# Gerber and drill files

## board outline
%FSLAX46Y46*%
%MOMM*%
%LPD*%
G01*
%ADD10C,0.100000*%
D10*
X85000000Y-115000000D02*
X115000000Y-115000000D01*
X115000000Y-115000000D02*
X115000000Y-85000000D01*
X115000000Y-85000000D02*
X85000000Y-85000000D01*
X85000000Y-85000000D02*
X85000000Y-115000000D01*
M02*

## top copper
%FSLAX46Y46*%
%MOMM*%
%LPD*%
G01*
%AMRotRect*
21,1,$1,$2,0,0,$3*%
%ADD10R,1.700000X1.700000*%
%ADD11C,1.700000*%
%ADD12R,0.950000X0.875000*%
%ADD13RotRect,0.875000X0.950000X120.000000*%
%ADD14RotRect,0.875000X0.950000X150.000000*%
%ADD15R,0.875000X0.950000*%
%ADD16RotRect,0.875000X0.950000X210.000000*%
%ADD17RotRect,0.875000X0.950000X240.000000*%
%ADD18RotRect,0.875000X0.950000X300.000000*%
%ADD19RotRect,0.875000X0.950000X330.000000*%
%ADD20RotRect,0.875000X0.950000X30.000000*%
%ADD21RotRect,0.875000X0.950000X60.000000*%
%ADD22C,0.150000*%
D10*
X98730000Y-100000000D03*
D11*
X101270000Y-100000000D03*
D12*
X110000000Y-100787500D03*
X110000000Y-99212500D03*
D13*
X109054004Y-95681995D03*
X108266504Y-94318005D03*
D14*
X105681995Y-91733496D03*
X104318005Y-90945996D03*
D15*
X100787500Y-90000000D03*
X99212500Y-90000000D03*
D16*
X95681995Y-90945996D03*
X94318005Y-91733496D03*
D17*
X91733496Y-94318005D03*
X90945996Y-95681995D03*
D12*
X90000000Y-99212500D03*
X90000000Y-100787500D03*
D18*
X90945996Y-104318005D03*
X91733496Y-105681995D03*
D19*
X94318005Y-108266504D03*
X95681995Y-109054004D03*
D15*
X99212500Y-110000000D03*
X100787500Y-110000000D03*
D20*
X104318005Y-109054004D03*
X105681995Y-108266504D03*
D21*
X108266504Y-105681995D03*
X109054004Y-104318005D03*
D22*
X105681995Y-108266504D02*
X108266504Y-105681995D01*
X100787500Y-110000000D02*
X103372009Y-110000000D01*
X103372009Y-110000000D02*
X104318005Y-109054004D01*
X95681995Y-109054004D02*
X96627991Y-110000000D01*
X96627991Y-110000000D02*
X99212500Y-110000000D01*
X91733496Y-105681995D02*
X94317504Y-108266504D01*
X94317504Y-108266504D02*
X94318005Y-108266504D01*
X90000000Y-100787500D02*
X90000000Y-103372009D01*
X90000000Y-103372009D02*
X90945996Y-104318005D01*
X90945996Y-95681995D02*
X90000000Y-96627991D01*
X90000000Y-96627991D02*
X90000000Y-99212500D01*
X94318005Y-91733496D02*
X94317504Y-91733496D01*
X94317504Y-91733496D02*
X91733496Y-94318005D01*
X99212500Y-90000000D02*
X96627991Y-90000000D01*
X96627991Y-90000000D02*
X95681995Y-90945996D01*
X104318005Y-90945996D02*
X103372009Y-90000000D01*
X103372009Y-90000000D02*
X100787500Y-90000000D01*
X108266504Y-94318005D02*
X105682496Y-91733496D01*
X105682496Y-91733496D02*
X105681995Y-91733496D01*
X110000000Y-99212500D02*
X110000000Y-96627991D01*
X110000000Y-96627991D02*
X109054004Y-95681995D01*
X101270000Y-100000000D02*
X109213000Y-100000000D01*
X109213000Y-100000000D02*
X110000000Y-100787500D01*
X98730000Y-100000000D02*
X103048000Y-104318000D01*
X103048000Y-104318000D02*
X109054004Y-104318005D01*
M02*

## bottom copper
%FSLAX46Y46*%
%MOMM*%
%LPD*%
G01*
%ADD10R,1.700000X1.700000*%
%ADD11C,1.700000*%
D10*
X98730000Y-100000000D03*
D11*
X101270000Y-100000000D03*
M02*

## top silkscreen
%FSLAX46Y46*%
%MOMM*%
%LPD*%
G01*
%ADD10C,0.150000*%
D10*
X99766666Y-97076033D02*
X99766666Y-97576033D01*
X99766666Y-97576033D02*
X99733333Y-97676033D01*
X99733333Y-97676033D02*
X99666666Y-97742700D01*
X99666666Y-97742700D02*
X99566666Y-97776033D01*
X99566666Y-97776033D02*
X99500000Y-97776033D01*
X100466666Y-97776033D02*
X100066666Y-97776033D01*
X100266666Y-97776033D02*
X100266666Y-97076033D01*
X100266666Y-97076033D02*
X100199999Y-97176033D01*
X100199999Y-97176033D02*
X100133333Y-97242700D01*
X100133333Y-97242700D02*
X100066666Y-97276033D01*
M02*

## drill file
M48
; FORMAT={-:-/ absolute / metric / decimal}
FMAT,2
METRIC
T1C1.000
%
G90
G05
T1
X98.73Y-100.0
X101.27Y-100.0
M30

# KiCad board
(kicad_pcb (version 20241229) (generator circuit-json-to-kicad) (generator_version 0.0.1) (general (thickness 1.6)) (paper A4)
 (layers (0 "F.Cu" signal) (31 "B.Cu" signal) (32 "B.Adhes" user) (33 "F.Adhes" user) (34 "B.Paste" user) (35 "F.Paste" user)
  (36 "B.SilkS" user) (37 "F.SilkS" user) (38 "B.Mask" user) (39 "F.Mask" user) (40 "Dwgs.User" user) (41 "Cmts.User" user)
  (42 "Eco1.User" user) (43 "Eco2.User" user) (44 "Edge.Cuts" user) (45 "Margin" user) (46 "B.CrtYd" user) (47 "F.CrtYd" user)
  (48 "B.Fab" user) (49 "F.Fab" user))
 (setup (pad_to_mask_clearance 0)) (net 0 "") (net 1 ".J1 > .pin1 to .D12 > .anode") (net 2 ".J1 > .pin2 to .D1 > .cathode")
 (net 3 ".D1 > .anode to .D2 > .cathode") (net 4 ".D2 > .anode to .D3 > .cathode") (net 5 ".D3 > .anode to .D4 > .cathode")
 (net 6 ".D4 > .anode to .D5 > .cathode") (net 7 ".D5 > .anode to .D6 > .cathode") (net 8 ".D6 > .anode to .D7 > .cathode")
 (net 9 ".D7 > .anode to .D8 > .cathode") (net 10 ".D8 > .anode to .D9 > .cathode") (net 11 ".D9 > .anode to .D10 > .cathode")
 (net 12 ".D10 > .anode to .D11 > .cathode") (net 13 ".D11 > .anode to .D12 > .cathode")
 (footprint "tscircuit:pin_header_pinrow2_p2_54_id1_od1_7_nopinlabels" (layer F.Cu) (at 100 100 0)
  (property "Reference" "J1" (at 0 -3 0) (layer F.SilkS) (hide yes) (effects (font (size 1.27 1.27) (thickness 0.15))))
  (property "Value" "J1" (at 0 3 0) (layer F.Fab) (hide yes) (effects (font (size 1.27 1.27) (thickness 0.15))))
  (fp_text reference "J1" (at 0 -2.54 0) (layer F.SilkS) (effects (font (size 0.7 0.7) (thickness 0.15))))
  (pad "1" thru_hole rect (at -1.27 0 0) (size 1.7 1.7) (drill 1) (layers *.Cu *.Mask) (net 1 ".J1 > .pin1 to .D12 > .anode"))
  (pad "2" thru_hole circle (at 1.27 0 0) (size 1.7 1.7) (drill 1) (layers *.Cu *.Mask) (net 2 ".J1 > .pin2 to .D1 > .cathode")))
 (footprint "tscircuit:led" (layer F.Cu) (at 110 100 90)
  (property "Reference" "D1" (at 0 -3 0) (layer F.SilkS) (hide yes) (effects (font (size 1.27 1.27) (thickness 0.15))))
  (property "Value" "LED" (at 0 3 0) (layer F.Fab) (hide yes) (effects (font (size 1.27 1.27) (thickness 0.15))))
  (pad "2" smd rect (at -0.7875 0 0) (size 0.95 0.875) (layers F.Cu F.Mask) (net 2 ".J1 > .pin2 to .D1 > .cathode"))
  (pad "1" smd rect (at 0.7875 0 0) (size 0.95 0.875) (layers F.Cu F.Mask) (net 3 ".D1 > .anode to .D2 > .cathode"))
  (pad "" smd rect (at -0.7875 0 0) (size 0.6649999999999999 0.6124999999999999) (layers F.Paste))
  (pad "" smd rect (at 0.7875 0 0) (size 0.6649999999999999 0.6124999999999999) (layers F.Paste)))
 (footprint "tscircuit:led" (layer F.Cu) (at 108.66025403784438 95 120)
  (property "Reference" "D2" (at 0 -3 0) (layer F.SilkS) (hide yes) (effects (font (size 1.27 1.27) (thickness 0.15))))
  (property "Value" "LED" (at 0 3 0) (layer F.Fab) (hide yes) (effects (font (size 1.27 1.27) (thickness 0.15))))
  (pad "2" smd rect (at -0.7874999999999996 0 120) (size 0.875 0.95) (layers F.Cu F.Mask) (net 3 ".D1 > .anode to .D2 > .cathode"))
  (pad "1" smd rect (at 0.7874999999999988 1.7763568394002505e-15 120) (size 0.875 0.95) (layers F.Cu F.Mask)
   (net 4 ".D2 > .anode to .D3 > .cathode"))
  (pad "" smd rect (at -0.7874999999999996 0 120) (size 0.6124999999999999 0.6649999999999999) (layers F.Paste))
  (pad "" smd rect (at 0.7874999999999988 1.7763568394002505e-15 120) (size 0.6124999999999999 0.6649999999999999) (layers F.Paste)))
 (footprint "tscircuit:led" (layer F.Cu) (at 105 91.33974596215562 150)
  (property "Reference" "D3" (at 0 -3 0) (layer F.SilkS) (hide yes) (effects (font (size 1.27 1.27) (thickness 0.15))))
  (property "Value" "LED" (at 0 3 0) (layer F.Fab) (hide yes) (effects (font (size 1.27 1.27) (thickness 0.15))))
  (pad "2" smd rect (at -0.7874999999999996 -1.7763568394002505e-15 150) (size 0.875 0.95) (layers F.Cu F.Mask)
   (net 4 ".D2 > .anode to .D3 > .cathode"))
  (pad "1" smd rect (at 0.7875000000000005 0 150) (size 0.875 0.95) (layers F.Cu F.Mask) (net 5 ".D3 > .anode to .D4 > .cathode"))
  (pad "" smd rect (at -0.7874999999999996 -1.7763568394002505e-15 150) (size 0.6124999999999999 0.6649999999999999) (layers F.Paste))
  (pad "" smd rect (at 0.7875000000000005 0 150) (size 0.6124999999999999 0.6649999999999999) (layers F.Paste)))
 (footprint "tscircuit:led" (layer F.Cu) (at 100 90 180)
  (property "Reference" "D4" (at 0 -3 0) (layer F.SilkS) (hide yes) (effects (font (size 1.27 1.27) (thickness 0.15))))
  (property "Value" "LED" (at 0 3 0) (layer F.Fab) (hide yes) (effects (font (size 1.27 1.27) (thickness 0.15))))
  (pad "2" smd rect (at -0.7875000000000001 0 0) (size 0.875 0.95) (layers F.Cu F.Mask) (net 5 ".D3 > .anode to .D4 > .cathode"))
  (pad "1" smd rect (at 0.7874999999999999 0 0) (size 0.875 0.95) (layers F.Cu F.Mask) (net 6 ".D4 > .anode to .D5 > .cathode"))
  (pad "" smd rect (at -0.7875000000000001 0 0) (size 0.6124999999999999 0.6649999999999999) (layers F.Paste))
  (pad "" smd rect (at 0.7874999999999999 0 0) (size 0.6124999999999999 0.6649999999999999) (layers F.Paste)))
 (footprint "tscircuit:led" (layer F.Cu) (at 95 91.3397459621556 209.99999999999997)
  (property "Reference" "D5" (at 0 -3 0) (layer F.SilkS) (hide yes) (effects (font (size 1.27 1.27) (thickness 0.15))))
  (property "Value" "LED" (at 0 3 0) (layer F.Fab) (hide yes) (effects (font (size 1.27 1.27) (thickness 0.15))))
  (pad "2" smd rect
   (at -0.7875000000000005 1.7763568394002505e-15 209.99999999999997) (size 0.875 0.95) (layers F.Cu F.Mask)
   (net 6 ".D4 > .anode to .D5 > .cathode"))
  (pad "1" smd rect
   (at 0.7875000000000005 -1.7763568394002505e-15 209.99999999999997) (size 0.875 0.95) (layers F.Cu F.Mask)
   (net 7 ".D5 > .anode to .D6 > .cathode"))
  (pad "" smd rect
   (at -0.7875000000000005 1.7763568394002505e-15 209.99999999999997) (size 0.6124999999999999 0.6649999999999999) (layers F.Paste))
  (pad "" smd rect
   (at 0.7875000000000005 -1.7763568394002505e-15 209.99999999999997) (size 0.6124999999999999 0.6649999999999999) (layers F.Paste)))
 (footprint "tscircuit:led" (layer F.Cu) (at 91.33974596215562 95 239.99999999999994)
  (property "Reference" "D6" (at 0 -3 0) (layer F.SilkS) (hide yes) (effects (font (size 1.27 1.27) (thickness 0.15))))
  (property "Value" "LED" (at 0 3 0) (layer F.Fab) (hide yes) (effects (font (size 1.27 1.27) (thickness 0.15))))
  (pad "2" smd rect (at -0.7875000000000005 0 239.99999999999994) (size 0.875 0.95) (layers F.Cu F.Mask)
   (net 7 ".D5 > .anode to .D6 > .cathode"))
  (pad "1" smd rect (at 0.7875000000000001 0 239.99999999999994) (size 0.875 0.95) (layers F.Cu F.Mask)
   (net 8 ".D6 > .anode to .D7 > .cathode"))
  (pad "" smd rect (at -0.7875000000000005 0 239.99999999999994) (size 0.6124999999999999 0.6649999999999999) (layers F.Paste))
  (pad "" smd rect (at 0.7875000000000001 0 239.99999999999994) (size 0.6124999999999999 0.6649999999999999) (layers F.Paste)))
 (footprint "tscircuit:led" (layer F.Cu) (at 90 100 270)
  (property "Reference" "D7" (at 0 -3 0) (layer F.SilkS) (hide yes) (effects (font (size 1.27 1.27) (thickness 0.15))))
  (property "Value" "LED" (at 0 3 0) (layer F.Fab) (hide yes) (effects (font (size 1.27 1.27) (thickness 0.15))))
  (pad "2" smd rect (at -0.7875 0 0) (size 0.95 0.875) (layers F.Cu F.Mask) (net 8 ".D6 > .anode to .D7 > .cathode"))
  (pad "1" smd rect (at 0.7875 0 0) (size 0.95 0.875) (layers F.Cu F.Mask) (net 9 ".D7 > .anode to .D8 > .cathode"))
  (pad "" smd rect (at -0.7875 0 0) (size 0.6649999999999999 0.6124999999999999) (layers F.Paste))
  (pad "" smd rect (at 0.7875 0 0) (size 0.6649999999999999 0.6124999999999999) (layers F.Paste)))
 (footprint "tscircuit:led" (layer F.Cu) (at 91.33974596215562 105 300)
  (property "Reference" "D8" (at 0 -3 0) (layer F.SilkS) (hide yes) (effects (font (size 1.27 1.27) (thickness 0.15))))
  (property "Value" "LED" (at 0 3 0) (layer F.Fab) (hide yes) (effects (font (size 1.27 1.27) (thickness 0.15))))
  (pad "2" smd rect (at -0.7875000000000001 0 300) (size 0.875 0.95) (layers F.Cu F.Mask) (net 9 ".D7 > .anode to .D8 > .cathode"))
  (pad "1" smd rect (at 0.7875000000000005 -1.7763568394002505e-15 300) (size 0.875 0.95) (layers F.Cu F.Mask)
   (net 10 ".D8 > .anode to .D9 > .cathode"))
  (pad "" smd rect (at -0.7875000000000001 0 300) (size 0.6124999999999999 0.6649999999999999) (layers F.Paste))
  (pad "" smd rect (at 0.7875000000000005 -1.7763568394002505e-15 300) (size 0.6124999999999999 0.6649999999999999) (layers F.Paste)))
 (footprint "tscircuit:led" (layer F.Cu) (at 95 108.66025403784438 330)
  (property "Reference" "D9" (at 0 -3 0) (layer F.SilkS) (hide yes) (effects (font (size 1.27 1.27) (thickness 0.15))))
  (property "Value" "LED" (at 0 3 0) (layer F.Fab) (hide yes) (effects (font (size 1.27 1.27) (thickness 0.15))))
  (pad "2" smd rect (at -0.7875000000000005 0 330) (size 0.875 0.95) (layers F.Cu F.Mask) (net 10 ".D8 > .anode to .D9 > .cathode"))
  (pad "1" smd rect (at 0.7875000000000005 0 330) (size 0.875 0.95) (layers F.Cu F.Mask) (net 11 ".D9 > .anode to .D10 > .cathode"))
  (pad "" smd rect (at -0.7875000000000005 0 330) (size 0.6124999999999999 0.6649999999999999) (layers F.Paste))
  (pad "" smd rect (at 0.7875000000000005 0 330) (size 0.6124999999999999 0.6649999999999999) (layers F.Paste)))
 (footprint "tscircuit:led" (layer F.Cu) (at 100 110 0)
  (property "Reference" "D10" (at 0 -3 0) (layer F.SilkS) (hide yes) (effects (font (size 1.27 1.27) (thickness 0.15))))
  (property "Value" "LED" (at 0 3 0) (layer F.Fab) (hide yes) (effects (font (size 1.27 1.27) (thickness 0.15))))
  (pad "2" smd rect (at -0.7875 0 0) (size 0.875 0.95) (layers F.Cu F.Mask) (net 11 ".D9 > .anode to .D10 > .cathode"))
  (pad "1" smd rect (at 0.7875 0 0) (size 0.875 0.95) (layers F.Cu F.Mask) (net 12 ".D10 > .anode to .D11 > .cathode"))
  (pad "" smd rect (at -0.7875 0 0) (size 0.6124999999999999 0.6649999999999999) (layers F.Paste))
  (pad "" smd rect (at 0.7875 0 0) (size 0.6124999999999999 0.6649999999999999) (layers F.Paste)))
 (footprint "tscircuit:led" (layer F.Cu) (at 105 108.66025403784438 30)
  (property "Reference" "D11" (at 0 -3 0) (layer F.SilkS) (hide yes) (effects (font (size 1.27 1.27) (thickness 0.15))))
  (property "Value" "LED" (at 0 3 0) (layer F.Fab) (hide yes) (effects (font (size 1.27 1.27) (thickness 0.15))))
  (pad "2" smd rect (at -0.7875000000000005 0 30) (size 0.875 0.95) (layers F.Cu F.Mask) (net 12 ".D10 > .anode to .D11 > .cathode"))
  (pad "1" smd rect (at 0.7875000000000005 -1.7763568394002505e-15 30) (size 0.875 0.95) (layers F.Cu F.Mask)
   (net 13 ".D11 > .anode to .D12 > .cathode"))
  (pad "" smd rect (at -0.7875000000000005 0 30) (size 0.6124999999999999 0.6649999999999999) (layers F.Paste))
  (pad "" smd rect (at 0.7875000000000005 -1.7763568394002505e-15 30) (size 0.6124999999999999 0.6649999999999999) (layers F.Paste)))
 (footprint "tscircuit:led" (layer F.Cu) (at 108.66025403784438 105 60)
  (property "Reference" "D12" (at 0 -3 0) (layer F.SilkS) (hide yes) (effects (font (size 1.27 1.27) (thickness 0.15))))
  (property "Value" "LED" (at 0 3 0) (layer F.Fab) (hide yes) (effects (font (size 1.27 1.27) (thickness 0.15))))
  (pad "2" smd rect (at -0.7874999999999996 0 60) (size 0.875 0.95) (layers F.Cu F.Mask) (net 13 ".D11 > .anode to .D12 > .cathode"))
  (pad "1" smd rect (at 0.7875000000000005 0 60) (size 0.875 0.95) (layers F.Cu F.Mask) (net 1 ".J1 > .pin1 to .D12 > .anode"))
  (pad "" smd rect (at -0.7874999999999996 0 60) (size 0.6124999999999999 0.6649999999999999) (layers F.Paste))
  (pad "" smd rect (at 0.7875000000000005 0 60) (size 0.6124999999999999 0.6649999999999999) (layers F.Paste)))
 (segment (start 105.68199500548025 108.26650403784438) (end 108.26650403784438 105.68199500548025) (width 0.15) (layer F.Cu) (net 13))
 (segment (start 100.7875 110) (end 103.37200903236415 110) (width 0.15) (layer F.Cu) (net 12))
 (segment (start 103.37200903236415 110) (end 104.31800499451975 109.05400403784438) (width 0.15) (layer F.Cu) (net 12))
 (segment (start 95.68199500548025 109.05400403784438) (end 96.62799096763585 110) (width 0.15) (layer F.Cu) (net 11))
 (segment (start 96.62799096763585 110) (end 99.21249999999999 110) (width 0.15) (layer F.Cu) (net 11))
 (segment (start 91.73349596215562 105.68199500548025) (end 94.31750403784439 108.26650403784438) (width 0.15) (layer F.Cu) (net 10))
 (segment (start 94.31750403784439 108.26650403784438) (end 94.31800499451975 108.26650403784438) (width 0.15) (layer F.Cu) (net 10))
 (segment (start 90 100.7875) (end 90 103.37200903236415) (width 0.15) (layer F.Cu) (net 9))
 (segment (start 90 103.37200903236415) (end 90.94599596215562 104.31800499451975) (width 0.15) (layer F.Cu) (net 9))
 (segment (start 90.9459959621556 95.68199500548025) (end 90 96.62799096763585) (width 0.15) (layer F.Cu) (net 8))
 (segment (start 90 96.62799096763585) (end 90 99.2125) (width 0.15) (layer F.Cu) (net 8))
 (segment (start 94.31800499451975 91.73349596215562) (end 94.31750403784439 91.73349596215562) (width 0.15) (layer F.Cu) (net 7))
 (segment (start 94.31750403784439 91.73349596215562) (end 91.73349596215562 94.31800499451975) (width 0.15) (layer F.Cu) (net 7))
 (segment (start 99.2125 90) (end 96.62799096763585 90) (width 0.15) (layer F.Cu) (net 6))
 (segment (start 96.62799096763585 90) (end 95.68199500548025 90.9459959621556) (width 0.15) (layer F.Cu) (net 6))
 (segment (start 104.31800499451975 90.94599596215562) (end 103.37200903236415 90) (width 0.15) (layer F.Cu) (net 5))
 (segment (start 103.37200903236415 90) (end 100.7875 90) (width 0.15) (layer F.Cu) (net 5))
 (segment (start 108.26650403784438 94.31800499451975) (end 105.68249596215561 91.73349596215562) (width 0.15) (layer F.Cu) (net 4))
 (segment (start 105.68249596215561 91.73349596215562) (end 105.68199500548025 91.73349596215562) (width 0.15) (layer F.Cu) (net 4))
 (segment (start 110 99.2125) (end 110 96.62799096763587) (width 0.15) (layer F.Cu) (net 3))
 (segment (start 110 96.62799096763587) (end 109.05400403784438 95.68199500548025) (width 0.15) (layer F.Cu) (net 3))
 (segment (start 101.27 100) (end 109.213 100) (width 0.15) (layer F.Cu) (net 2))
 (segment (start 109.213 100) (end 110 100.7875) (width 0.15) (layer F.Cu) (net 2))
 (segment (start 98.73 100) (end 103.048 104.318) (width 0.15) (layer F.Cu) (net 1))
 (segment (start 103.048 104.318) (end 109.05400403784438 104.31800499451975) (width 0.15) (layer F.Cu) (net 1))
 (gr_line (start 85 115) (end 115 115) (width 0.1) (layer Edge.Cuts))
 (gr_line (start 115 115) (end 115 85) (width 0.1) (layer Edge.Cuts))
 (gr_line (start 115 85) (end 85 85) (width 0.1) (layer Edge.Cuts))
 (gr_line (start 85 85) (end 85 115) (width 0.1) (layer Edge.Cuts)))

